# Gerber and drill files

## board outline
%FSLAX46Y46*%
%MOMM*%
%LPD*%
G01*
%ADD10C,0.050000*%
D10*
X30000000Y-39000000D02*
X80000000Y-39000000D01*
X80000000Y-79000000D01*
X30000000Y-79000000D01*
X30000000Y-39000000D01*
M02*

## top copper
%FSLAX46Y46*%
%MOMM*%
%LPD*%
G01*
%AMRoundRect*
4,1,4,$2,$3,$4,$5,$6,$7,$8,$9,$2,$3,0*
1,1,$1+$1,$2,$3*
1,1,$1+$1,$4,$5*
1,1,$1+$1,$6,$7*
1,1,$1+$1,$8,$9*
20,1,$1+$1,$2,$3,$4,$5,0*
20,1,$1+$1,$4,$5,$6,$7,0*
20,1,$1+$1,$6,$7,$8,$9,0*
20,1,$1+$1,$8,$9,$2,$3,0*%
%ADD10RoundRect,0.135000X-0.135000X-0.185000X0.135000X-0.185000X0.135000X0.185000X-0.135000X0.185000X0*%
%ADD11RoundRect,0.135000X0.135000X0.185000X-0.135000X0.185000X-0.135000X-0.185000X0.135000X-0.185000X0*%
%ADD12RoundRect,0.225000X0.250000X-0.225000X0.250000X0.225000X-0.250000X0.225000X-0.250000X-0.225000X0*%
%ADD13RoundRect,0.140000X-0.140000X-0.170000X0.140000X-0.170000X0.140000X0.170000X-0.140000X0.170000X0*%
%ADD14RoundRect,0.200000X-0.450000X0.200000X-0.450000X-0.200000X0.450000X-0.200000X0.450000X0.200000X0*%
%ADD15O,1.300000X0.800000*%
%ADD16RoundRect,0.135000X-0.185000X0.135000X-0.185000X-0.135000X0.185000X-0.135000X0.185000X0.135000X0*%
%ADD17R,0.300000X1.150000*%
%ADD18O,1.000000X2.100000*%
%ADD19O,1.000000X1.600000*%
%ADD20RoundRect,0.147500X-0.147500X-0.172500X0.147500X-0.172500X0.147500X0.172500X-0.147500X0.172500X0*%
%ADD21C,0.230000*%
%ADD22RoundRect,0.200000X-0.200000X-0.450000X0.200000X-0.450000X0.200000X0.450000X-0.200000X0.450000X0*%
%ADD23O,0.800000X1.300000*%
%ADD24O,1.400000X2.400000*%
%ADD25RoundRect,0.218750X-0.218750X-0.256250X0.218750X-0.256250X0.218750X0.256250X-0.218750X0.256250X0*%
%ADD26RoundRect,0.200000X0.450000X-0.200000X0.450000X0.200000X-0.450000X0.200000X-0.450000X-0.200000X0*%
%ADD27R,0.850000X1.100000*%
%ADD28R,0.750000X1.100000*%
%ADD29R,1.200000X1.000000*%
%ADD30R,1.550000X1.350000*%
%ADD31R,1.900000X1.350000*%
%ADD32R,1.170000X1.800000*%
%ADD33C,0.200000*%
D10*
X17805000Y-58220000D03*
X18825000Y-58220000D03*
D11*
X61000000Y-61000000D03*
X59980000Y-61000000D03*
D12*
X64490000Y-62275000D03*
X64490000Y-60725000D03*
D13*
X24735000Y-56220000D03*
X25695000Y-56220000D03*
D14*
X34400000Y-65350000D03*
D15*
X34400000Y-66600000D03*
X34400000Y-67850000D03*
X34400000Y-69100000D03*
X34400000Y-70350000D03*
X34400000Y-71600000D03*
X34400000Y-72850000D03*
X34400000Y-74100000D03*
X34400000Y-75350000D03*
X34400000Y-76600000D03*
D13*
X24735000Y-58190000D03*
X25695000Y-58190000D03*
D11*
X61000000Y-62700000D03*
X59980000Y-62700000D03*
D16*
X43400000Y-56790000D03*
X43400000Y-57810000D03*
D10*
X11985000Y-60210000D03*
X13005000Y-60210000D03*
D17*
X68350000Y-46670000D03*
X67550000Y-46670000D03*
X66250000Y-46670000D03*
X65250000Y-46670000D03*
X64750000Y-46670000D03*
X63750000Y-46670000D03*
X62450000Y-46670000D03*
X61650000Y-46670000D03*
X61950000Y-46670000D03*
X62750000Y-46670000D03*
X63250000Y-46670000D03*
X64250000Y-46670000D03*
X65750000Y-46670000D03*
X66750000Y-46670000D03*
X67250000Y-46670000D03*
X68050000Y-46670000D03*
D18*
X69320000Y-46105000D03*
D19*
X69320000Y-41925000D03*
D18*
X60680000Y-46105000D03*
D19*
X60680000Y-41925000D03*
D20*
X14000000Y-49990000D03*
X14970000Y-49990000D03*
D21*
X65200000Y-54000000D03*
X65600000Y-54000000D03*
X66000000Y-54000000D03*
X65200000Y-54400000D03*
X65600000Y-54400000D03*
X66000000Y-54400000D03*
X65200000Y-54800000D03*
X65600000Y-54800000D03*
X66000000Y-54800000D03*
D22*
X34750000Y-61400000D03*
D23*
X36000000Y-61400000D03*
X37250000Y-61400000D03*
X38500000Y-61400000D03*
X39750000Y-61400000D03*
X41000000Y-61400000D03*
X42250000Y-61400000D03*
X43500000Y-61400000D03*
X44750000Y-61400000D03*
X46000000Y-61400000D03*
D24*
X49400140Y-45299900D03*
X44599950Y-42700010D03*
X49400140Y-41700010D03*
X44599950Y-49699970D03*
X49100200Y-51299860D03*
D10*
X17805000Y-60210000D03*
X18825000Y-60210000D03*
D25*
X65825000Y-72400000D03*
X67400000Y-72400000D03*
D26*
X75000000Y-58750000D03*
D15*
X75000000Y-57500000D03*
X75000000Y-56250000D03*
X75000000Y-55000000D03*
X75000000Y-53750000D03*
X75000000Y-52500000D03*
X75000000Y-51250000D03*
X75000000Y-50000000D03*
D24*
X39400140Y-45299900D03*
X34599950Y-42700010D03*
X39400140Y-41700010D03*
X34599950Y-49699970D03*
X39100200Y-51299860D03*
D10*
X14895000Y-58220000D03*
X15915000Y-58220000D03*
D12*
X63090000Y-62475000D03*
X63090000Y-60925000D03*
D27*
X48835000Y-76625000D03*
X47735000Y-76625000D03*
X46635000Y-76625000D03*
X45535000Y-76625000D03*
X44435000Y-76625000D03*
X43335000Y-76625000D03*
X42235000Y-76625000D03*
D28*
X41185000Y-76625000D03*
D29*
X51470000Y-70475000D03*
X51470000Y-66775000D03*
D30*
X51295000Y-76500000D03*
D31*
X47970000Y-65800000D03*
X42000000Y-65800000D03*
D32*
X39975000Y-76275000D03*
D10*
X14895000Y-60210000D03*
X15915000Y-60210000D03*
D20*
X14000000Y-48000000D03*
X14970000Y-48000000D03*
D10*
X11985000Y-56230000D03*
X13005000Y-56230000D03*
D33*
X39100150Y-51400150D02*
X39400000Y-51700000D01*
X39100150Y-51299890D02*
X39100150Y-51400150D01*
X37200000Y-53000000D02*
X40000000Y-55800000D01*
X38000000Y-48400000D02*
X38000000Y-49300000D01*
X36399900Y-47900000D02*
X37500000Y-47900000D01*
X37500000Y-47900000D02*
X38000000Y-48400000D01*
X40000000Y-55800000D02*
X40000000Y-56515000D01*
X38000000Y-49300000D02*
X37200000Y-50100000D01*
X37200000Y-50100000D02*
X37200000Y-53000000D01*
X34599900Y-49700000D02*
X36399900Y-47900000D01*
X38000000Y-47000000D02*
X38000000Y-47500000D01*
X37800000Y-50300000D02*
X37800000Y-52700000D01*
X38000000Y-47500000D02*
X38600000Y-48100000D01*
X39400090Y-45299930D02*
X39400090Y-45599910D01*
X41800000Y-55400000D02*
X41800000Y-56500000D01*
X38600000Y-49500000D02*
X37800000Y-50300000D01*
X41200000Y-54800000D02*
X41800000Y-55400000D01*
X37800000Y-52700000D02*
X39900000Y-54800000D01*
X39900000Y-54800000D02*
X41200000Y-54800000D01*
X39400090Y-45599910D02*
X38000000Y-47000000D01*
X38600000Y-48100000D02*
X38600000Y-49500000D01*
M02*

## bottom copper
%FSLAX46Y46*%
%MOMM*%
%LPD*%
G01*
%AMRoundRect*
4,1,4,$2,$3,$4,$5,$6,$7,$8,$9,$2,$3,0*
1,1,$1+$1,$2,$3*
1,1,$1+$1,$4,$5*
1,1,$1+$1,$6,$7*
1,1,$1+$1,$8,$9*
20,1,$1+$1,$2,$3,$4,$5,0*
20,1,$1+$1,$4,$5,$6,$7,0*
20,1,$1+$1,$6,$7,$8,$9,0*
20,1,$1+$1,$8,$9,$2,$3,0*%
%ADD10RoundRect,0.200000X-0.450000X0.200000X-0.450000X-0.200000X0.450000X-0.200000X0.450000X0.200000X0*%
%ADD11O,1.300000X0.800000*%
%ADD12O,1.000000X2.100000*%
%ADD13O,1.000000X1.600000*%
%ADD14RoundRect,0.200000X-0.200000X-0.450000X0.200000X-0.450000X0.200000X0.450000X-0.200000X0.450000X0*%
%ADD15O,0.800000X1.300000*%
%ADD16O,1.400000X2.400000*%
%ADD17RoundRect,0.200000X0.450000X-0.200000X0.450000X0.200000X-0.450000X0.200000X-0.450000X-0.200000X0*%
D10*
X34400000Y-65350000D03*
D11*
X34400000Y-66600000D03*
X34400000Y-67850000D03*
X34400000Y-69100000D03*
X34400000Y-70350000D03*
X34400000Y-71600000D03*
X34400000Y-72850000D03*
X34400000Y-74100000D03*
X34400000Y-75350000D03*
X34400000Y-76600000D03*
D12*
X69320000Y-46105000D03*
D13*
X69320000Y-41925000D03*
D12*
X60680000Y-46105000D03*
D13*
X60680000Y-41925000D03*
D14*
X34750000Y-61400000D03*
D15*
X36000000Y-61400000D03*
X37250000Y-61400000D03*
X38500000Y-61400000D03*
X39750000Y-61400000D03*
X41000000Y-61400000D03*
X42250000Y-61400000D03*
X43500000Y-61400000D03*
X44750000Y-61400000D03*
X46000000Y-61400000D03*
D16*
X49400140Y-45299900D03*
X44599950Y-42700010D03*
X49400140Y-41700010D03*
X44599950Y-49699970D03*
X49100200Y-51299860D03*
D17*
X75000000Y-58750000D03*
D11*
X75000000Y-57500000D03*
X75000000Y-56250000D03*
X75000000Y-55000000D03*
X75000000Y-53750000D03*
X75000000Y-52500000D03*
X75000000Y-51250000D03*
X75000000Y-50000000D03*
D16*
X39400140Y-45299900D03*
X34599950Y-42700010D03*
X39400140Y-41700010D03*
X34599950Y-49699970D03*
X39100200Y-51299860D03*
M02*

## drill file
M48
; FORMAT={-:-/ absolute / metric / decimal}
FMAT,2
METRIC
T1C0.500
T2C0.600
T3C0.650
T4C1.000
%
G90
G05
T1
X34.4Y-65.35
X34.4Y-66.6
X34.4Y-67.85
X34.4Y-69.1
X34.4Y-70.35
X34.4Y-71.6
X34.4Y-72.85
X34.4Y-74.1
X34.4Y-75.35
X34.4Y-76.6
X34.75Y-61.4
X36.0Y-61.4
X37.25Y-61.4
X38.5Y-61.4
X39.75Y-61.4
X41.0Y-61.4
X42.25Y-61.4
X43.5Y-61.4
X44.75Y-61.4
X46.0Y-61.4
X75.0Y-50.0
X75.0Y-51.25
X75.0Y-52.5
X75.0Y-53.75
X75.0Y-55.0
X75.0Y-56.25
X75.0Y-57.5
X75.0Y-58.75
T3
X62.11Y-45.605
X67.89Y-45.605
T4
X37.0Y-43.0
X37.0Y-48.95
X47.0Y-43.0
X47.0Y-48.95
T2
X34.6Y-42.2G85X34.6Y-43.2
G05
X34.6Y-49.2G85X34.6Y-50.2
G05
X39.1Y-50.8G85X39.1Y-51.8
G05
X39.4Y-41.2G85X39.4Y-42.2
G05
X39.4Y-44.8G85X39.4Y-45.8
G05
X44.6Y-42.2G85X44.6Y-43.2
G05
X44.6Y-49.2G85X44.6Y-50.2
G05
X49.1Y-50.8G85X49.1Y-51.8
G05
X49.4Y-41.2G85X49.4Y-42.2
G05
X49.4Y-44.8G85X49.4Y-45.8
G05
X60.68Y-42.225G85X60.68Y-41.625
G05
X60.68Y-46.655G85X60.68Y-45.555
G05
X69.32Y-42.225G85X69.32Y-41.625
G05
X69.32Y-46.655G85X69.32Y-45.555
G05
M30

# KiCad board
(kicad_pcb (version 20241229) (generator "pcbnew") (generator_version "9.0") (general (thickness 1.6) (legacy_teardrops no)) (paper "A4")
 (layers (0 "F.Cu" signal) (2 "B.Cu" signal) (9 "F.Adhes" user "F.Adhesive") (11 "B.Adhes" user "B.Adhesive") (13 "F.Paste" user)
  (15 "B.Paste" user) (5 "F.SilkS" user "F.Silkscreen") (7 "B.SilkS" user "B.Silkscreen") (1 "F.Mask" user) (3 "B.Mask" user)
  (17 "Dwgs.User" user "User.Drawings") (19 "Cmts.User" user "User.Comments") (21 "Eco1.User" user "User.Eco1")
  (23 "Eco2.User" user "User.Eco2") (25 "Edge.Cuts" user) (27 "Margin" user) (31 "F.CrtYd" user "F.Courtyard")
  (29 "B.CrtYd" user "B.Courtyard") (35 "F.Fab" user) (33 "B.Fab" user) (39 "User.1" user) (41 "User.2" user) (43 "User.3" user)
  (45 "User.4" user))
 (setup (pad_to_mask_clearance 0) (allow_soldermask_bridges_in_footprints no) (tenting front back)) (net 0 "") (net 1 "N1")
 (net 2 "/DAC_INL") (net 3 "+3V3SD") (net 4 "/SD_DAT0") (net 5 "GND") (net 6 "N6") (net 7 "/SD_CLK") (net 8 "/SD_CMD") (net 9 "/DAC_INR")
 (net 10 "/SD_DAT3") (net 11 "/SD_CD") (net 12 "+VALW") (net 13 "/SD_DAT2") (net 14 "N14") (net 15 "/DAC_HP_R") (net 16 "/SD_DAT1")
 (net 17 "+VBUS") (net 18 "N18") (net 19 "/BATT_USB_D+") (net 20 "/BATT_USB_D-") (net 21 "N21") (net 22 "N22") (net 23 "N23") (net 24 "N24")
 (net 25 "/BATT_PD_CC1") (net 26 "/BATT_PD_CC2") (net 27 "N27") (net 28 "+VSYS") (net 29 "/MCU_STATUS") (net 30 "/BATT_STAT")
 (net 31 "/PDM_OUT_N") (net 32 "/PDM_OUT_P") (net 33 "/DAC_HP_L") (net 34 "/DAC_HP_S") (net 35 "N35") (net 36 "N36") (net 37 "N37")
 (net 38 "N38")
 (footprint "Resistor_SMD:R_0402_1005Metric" (layer "F.Cu") (at 18.315 58.22)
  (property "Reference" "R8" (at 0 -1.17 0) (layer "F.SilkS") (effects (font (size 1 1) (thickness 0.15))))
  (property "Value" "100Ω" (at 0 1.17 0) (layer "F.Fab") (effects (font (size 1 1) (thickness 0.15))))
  (pad "1" smd roundrect (at -0.51 0) (size 0.54 0.64) (layers "F.Cu" "F.Mask" "F.Paste") (roundrect_rratio 0.25) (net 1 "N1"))
  (pad "2" smd roundrect (at 0.51 0) (size 0.54 0.64) (layers "F.Cu" "F.Mask" "F.Paste") (roundrect_rratio 0.25) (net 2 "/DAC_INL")))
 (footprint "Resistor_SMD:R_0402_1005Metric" (layer "F.Cu") (at 60.49 61 180)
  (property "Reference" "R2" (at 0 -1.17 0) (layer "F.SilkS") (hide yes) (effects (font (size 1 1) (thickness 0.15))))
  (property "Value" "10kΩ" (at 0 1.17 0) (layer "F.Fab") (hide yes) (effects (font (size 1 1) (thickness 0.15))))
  (pad "1" smd roundrect (at -0.51 0 180) (size 0.54 0.64) (layers "F.Cu" "F.Mask" "F.Paste") (roundrect_rratio 0.25) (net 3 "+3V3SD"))
  (pad "2" smd roundrect (at 0.51 0 180) (size 0.54 0.64) (layers "F.Cu" "F.Mask" "F.Paste") (roundrect_rratio 0.25) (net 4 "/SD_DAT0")))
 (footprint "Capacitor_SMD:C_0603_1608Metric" (layer "F.Cu") (at 64.49 61.5 90)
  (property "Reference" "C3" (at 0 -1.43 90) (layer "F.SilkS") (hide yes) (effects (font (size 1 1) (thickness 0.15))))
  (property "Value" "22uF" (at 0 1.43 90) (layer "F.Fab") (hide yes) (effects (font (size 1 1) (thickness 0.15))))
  (pad "1" smd roundrect (at -0.775 0 90) (size 0.9 0.95) (layers "F.Cu" "F.Mask" "F.Paste") (roundrect_rratio 0.25) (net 3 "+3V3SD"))
  (pad "2" smd roundrect (at 0.775 0 90) (size 0.9 0.95) (layers "F.Cu" "F.Mask" "F.Paste") (roundrect_rratio 0.25) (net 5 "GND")))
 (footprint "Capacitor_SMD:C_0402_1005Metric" (layer "F.Cu") (at 25.215 56.22)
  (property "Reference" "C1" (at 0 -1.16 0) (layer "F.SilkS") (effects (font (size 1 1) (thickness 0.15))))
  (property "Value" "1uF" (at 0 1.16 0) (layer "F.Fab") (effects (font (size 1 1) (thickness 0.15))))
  (pad "1" smd roundrect (at -0.48 0) (size 0.56 0.62) (layers "F.Cu" "F.Mask" "F.Paste") (roundrect_rratio 0.25) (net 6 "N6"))
  (pad "2" smd roundrect (at 0.48 0) (size 0.56 0.62) (layers "F.Cu" "F.Mask" "F.Paste") (roundrect_rratio 0.25) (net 5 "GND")))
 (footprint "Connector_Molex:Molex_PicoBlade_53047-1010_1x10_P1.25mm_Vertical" (layer "F.Cu") (at 34.4 65.35 -90)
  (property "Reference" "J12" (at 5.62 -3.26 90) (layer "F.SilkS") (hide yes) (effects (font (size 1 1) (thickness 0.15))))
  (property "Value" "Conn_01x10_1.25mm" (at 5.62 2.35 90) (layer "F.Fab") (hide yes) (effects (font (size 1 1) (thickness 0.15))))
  (pad "1" thru_hole roundrect (at 0 0 270) (size 0.8 1.3) (drill 0.5) (layers "*.Cu" "*.Mask") (remove_unused_layers no)
   (roundrect_rratio 0.25) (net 5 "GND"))
  (pad "2" thru_hole oval (at 1.25 0 270) (size 0.8 1.3) (drill 0.5) (layers "*.Cu" "*.Mask") (remove_unused_layers no) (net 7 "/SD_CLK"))
  (pad "3" thru_hole oval (at 2.5 0 270) (size 0.8 1.3) (drill 0.5) (layers "*.Cu" "*.Mask") (remove_unused_layers no) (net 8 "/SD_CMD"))
  (pad "4" thru_hole oval (at 3.75 0 270) (size 0.8 1.3) (drill 0.5) (layers "*.Cu" "*.Mask") (remove_unused_layers no) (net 3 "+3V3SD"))
  (pad "5" thru_hole oval (at 5 0 270) (size 0.8 1.3) (drill 0.5) (layers "*.Cu" "*.Mask") (remove_unused_layers no) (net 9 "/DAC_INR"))
  (pad "6" thru_hole oval (at 6.25 0 270) (size 0.8 1.3) (drill 0.5) (layers "*.Cu" "*.Mask") (remove_unused_layers no) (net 2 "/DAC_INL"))
  (pad "7" thru_hole oval (at 7.5 0 270) (size 0.8 1.3) (drill 0.5) (layers "*.Cu" "*.Mask") (remove_unused_layers no) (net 5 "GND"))
  (pad "8" thru_hole oval (at 8.75 0 270) (size 0.8 1.3) (drill 0.5) (layers "*.Cu" "*.Mask") (remove_unused_layers no) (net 4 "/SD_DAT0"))
  (pad "9" thru_hole oval (at 10 0 270) (size 0.8 1.3) (drill 0.5) (layers "*.Cu" "*.Mask") (remove_unused_layers no) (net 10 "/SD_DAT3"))
  (pad "10" thru_hole oval (at 11.25 0 270) (size 0.8 1.3) (drill 0.5) (layers "*.Cu" "*.Mask") (remove_unused_layers no) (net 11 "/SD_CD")))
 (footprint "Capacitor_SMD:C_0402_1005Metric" (layer "F.Cu") (at 25.215 58.19)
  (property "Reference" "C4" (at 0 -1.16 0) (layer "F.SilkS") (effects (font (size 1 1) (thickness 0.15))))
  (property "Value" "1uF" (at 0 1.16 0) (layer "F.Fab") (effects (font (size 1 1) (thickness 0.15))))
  (pad "1" smd roundrect (at -0.48 0) (size 0.56 0.62) (layers "F.Cu" "F.Mask" "F.Paste") (roundrect_rratio 0.25) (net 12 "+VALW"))
  (pad "2" smd roundrect (at 0.48 0) (size 0.56 0.62) (layers "F.Cu" "F.Mask" "F.Paste") (roundrect_rratio 0.25) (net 5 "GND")))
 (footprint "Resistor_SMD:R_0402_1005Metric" (layer "F.Cu") (at 60.49 62.7 180)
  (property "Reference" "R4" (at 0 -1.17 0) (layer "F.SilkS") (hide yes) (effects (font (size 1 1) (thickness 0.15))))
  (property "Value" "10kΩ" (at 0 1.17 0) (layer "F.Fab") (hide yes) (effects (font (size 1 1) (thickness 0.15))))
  (pad "1" smd roundrect (at -0.51 0 180) (size 0.54 0.64) (layers "F.Cu" "F.Mask" "F.Paste") (roundrect_rratio 0.25) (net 3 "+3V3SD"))
  (pad "2" smd roundrect (at 0.51 0 180) (size 0.54 0.64) (layers "F.Cu" "F.Mask" "F.Paste") (roundrect_rratio 0.25) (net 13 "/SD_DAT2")))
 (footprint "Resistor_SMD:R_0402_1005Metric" (layer "F.Cu") (at 43.4 57.3 -90)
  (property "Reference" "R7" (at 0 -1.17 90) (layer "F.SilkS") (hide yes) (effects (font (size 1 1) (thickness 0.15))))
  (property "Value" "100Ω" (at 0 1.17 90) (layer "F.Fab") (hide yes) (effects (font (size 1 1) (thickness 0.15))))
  (pad "1" smd roundrect (at -0.51 0 270) (size 0.54 0.64) (layers "F.Cu" "F.Mask" "F.Paste") (roundrect_rratio 0.25) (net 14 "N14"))
  (pad "2" smd roundrect (at 0.51 0 270) (size 0.54 0.64) (layers "F.Cu" "F.Mask" "F.Paste") (roundrect_rratio 0.25) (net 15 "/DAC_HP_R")))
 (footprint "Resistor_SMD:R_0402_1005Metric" (layer "F.Cu") (at 12.495 60.21)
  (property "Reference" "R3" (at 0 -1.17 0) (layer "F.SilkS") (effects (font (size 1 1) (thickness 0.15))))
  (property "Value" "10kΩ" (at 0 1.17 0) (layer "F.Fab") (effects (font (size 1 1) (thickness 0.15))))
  (pad "1" smd roundrect (at -0.51 0) (size 0.54 0.64) (layers "F.Cu" "F.Mask" "F.Paste") (roundrect_rratio 0.25) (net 3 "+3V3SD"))
  (pad "2" smd roundrect (at 0.51 0) (size 0.54 0.64) (layers "F.Cu" "F.Mask" "F.Paste") (roundrect_rratio 0.25) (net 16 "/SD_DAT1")))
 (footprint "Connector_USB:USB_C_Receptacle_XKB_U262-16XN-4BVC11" (layer "F.Cu") (at 65 43 180)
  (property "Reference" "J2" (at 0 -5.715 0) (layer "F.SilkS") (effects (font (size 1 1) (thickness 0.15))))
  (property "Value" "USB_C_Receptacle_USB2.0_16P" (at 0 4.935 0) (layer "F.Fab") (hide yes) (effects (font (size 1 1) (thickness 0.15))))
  (pad "" np_thru_hole circle (at -2.89 -2.605 180) (size 0.65 0.65) (drill 0.65) (layers "*.Cu" "*.Mask"))
  (pad "" np_thru_hole circle (at 2.89 -2.605 180) (size 0.65 0.65) (drill 0.65) (layers "*.Cu" "*.Mask"))
  (pad "A1" smd rect (at -3.35 -3.67 180) (size 0.3 1.15) (layers "F.Cu" "F.Mask" "F.Paste") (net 5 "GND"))
  (pad "A4" smd rect (at -2.55 -3.67 180) (size 0.3 1.15) (layers "F.Cu" "F.Mask" "F.Paste") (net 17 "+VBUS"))
  (pad "A5" smd rect (at -1.25 -3.67 180) (size 0.3 1.15) (layers "F.Cu" "F.Mask" "F.Paste") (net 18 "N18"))
  (pad "A6" smd rect (at -0.25 -3.67 180) (size 0.3 1.15) (layers "F.Cu" "F.Mask" "F.Paste") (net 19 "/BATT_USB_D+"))
  (pad "A7" smd rect (at 0.25 -3.67 180) (size 0.3 1.15) (layers "F.Cu" "F.Mask" "F.Paste") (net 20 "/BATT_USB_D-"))
  (pad "A8" smd rect (at 1.25 -3.67 180) (size 0.3 1.15) (layers "F.Cu" "F.Mask" "F.Paste") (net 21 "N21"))
  (pad "A9" smd rect (at 2.55 -3.67 180) (size 0.3 1.15) (layers "F.Cu" "F.Mask" "F.Paste") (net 17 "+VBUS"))
  (pad "A12" smd rect (at 3.35 -3.67 180) (size 0.3 1.15) (layers "F.Cu" "F.Mask" "F.Paste") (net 5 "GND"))
  (pad "B1" smd rect (at 3.05 -3.67 180) (size 0.3 1.15) (layers "F.Cu" "F.Mask" "F.Paste") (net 5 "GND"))
  (pad "B4" smd rect (at 2.25 -3.67 180) (size 0.3 1.15) (layers "F.Cu" "F.Mask" "F.Paste") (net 17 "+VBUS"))
  (pad "B5" smd rect (at 1.75 -3.67 180) (size 0.3 1.15) (layers "F.Cu" "F.Mask" "F.Paste") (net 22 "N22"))
  (pad "B6" smd rect (at 0.75 -3.67 180) (size 0.3 1.15) (layers "F.Cu" "F.Mask" "F.Paste") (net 19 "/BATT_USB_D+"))
  (pad "B7" smd rect (at -0.75 -3.67 180) (size 0.3 1.15) (layers "F.Cu" "F.Mask" "F.Paste") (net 20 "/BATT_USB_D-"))
  (pad "B8" smd rect (at -1.75 -3.67 180) (size 0.3 1.15) (layers "F.Cu" "F.Mask" "F.Paste") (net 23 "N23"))
  (pad "B9" smd rect (at -2.25 -3.67 180) (size 0.3 1.15) (layers "F.Cu" "F.Mask" "F.Paste") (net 17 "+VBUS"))
  (pad "B12" smd rect (at -3.05 -3.67 180) (size 0.3 1.15) (layers "F.Cu" "F.Mask" "F.Paste") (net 5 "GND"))
  (pad "S1" thru_hole oval (at -4.32 -3.105 180) (size 1 2.1) (drill oval 0.6 1.7) (layers "*.Cu" "*.Mask") (remove_unused_layers no)
   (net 5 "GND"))
  (pad "S1" thru_hole oval (at -4.32 1.075 180) (size 1 1.6) (drill oval 0.6 1.2) (layers "*.Cu" "*.Mask") (remove_unused_layers no)
   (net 5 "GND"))
  (pad "S1" thru_hole oval (at 4.32 -3.105 180) (size 1 2.1) (drill oval 0.6 1.7) (layers "*.Cu" "*.Mask") (remove_unused_layers no)
   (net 5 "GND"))
  (pad "S1" thru_hole oval (at 4.32 1.075 180) (size 1 1.6) (drill oval 0.6 1.2) (layers "*.Cu" "*.Mask") (remove_unused_layers no)
   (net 5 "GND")))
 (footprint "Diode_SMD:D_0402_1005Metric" (layer "F.Cu") (at 14.485 49.99)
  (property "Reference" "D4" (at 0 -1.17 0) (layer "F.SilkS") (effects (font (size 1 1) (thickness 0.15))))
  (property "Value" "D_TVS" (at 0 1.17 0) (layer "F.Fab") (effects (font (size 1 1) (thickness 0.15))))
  (pad "1" smd roundrect (at -0.485 0) (size 0.59 0.64) (layers "F.Cu" "F.Mask" "F.Paste") (roundrect_rratio 0.25) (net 5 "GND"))
  (pad "2" smd roundrect (at 0.485 0) (size 0.59 0.64) (layers "F.Cu" "F.Mask" "F.Paste") (roundrect_rratio 0.25) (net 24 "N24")))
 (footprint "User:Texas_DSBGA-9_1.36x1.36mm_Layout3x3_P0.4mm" (layer "F.Cu") (at 65.6 54.4)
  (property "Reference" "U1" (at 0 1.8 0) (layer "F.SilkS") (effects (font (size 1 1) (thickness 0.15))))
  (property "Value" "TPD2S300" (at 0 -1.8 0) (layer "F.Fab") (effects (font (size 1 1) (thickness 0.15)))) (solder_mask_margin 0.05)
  (pad "A1" smd circle (at -0.4 -0.4) (size 0.23 0.23) (layers "F.Cu" "F.Paste") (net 18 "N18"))
  (pad "A2" smd circle (at 0 -0.4) (size 0.23 0.23) (layers "F.Cu" "F.Paste") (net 6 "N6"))
  (pad "A3" smd circle (at 0.4 -0.4) (size 0.23 0.23) (layers "F.Cu" "F.Paste") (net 22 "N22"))
  (pad "B1" smd circle (at -0.4 0) (size 0.23 0.23) (layers "F.Cu" "F.Paste") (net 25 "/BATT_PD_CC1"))
  (pad "B2" smd circle (at 0 0) (size 0.23 0.23) (layers "F.Cu" "F.Paste") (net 5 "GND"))
  (pad "B3" smd circle (at 0.4 0) (size 0.23 0.23) (layers "F.Cu" "F.Paste") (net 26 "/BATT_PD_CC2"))
  (pad "C1" smd circle (at -0.4 0.4) (size 0.23 0.23) (layers "F.Cu" "F.Paste") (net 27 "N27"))
  (pad "C2" smd circle (at 0 0.4) (size 0.23 0.23) (layers "F.Cu" "F.Paste") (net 12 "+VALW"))
  (pad "C3" smd circle (at 0.4 0.4) (size 0.23 0.23) (layers "F.Cu" "F.Paste") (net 12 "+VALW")))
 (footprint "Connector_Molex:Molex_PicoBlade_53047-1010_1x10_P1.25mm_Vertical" (layer "F.Cu") (at 34.75 61.4)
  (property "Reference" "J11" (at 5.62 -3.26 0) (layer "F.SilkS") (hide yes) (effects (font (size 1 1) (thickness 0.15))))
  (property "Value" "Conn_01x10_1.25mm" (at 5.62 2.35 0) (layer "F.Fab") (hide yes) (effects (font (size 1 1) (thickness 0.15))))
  (pad "1" thru_hole roundrect (at 0 0) (size 0.8 1.3) (drill 0.5) (layers "*.Cu" "*.Mask") (remove_unused_layers no)
   (roundrect_rratio 0.25) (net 5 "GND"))
  (pad "2" thru_hole oval (at 1.25 0) (size 0.8 1.3) (drill 0.5) (layers "*.Cu" "*.Mask") (remove_unused_layers no) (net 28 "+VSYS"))
  (pad "3" thru_hole oval (at 2.5 0) (size 0.8 1.3) (drill 0.5) (layers "*.Cu" "*.Mask") (remove_unused_layers no) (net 12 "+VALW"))
  (pad "4" thru_hole oval (at 3.75 0) (size 0.8 1.3) (drill 0.5) (layers "*.Cu" "*.Mask") (remove_unused_layers no) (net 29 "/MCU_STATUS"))
  (pad "5" thru_hole oval (at 5 0) (size 0.8 1.3) (drill 0.5) (layers "*.Cu" "*.Mask") (remove_unused_layers no) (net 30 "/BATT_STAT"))
  (pad "6" thru_hole oval (at 6.25 0) (size 0.8 1.3) (drill 0.5) (layers "*.Cu" "*.Mask") (remove_unused_layers no) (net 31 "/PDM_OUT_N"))
  (pad "7" thru_hole oval (at 7.5 0) (size 0.8 1.3) (drill 0.5) (layers "*.Cu" "*.Mask") (remove_unused_layers no) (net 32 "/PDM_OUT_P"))
  (pad "8" thru_hole oval (at 8.75 0) (size 0.8 1.3) (drill 0.5) (layers "*.Cu" "*.Mask") (remove_unused_layers no) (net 15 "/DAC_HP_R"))
  (pad "9" thru_hole oval (at 10 0) (size 0.8 1.3) (drill 0.5) (layers "*.Cu" "*.Mask") (remove_unused_layers no) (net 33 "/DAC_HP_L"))
  (pad "10" thru_hole oval (at 11.25 0) (size 0.8 1.3) (drill 0.5) (layers "*.Cu" "*.Mask") (remove_unused_layers no) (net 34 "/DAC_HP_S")))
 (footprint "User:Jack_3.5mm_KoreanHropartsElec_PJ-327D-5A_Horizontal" (layer "F.Cu") (at 47 46.5)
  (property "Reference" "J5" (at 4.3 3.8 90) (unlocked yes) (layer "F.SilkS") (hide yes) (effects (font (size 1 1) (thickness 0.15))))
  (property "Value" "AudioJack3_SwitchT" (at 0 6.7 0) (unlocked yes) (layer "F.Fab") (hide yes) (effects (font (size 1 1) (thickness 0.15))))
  (pad "" np_thru_hole circle (at 0 -3.5) (size 1 1) (drill 1) (layers "*.Cu" "*.Mask"))
  (pad "" np_thru_hole circle (at 0 2.45) (size 1 1) (drill 1) (layers "*.Cu" "*.Mask"))
  (pad "R" thru_hole oval (at 2.40009 -1.20007) (size 1.4 2.4) (drill oval 0.6 1.6 (offset 0.00005 -0.00003)) (layers "*.Cu" "*.Mask")
   (remove_unused_layers no) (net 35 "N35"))
  (pad "S" thru_hole oval (at -2.4001 -3.79996) (size 1.4 2.4) (drill oval 0.6 1.6 (offset 0.00005 -0.00003)) (layers "*.Cu" "*.Mask")
   (remove_unused_layers no) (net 5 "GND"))
  (pad "S" thru_hole oval (at 2.40009 -4.79996) (size 1.4 2.4) (drill oval 0.6 1.6 (offset 0.00005 -0.00003)) (layers "*.Cu" "*.Mask")
   (remove_unused_layers no) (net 5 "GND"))
  (pad "T" thru_hole oval (at -2.4001 3.2) (size 1.4 2.4) (drill oval 0.6 1.6 (offset 0.00005 -0.00003)) (layers "*.Cu" "*.Mask")
   (remove_unused_layers no) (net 1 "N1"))
  (pad "TN" thru_hole oval (at 2.10015 4.79989) (size 1.4 2.4) (drill oval 0.6 1.6 (offset 0.00005 -0.00003)) (layers "*.Cu" "*.Mask")
   (remove_unused_layers no) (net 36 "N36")))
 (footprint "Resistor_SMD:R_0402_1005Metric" (layer "F.Cu") (at 18.315 60.21)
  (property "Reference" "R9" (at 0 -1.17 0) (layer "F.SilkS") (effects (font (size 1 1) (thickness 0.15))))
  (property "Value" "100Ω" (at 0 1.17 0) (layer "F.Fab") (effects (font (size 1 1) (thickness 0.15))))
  (pad "1" smd roundrect (at -0.51 0) (size 0.54 0.64) (layers "F.Cu" "F.Mask" "F.Paste") (roundrect_rratio 0.25) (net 35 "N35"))
  (pad "2" smd roundrect (at 0.51 0) (size 0.54 0.64) (layers "F.Cu" "F.Mask" "F.Paste") (roundrect_rratio 0.25) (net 9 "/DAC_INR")))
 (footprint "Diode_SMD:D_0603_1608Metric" (layer "F.Cu") (at 66.6125 72.4)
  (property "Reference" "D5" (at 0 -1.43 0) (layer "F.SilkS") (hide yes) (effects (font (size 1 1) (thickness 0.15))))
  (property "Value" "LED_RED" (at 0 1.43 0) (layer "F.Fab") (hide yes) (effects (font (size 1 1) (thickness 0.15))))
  (pad "1" smd roundrect (at -0.7875 0) (size 0.875 0.95) (layers "F.Cu" "F.Mask" "F.Paste") (roundrect_rratio 0.25) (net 30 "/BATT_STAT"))
  (pad "2" smd roundrect (at 0.7875 0) (size 0.875 0.95) (layers "F.Cu" "F.Mask" "F.Paste") (roundrect_rratio 0.25) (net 12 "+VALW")))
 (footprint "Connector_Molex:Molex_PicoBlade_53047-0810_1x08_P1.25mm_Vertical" (layer "F.Cu") (at 75 58.75 90)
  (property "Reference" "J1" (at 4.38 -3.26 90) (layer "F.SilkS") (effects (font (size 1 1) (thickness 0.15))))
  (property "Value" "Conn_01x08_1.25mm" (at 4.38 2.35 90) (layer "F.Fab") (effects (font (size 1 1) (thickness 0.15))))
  (pad "1" thru_hole roundrect (at 0 0 90) (size 0.8 1.3) (drill 0.5) (layers "*.Cu" "*.Mask") (remove_unused_layers no)
   (roundrect_rratio 0.25) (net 17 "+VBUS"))
  (pad "2" thru_hole oval (at 1.25 0 90) (size 0.8 1.3) (drill 0.5) (layers "*.Cu" "*.Mask") (remove_unused_layers no) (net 17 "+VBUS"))
  (pad "3" thru_hole oval (at 2.5 0 90) (size 0.8 1.3) (drill 0.5) (layers "*.Cu" "*.Mask") (remove_unused_layers no) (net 5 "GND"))
  (pad "4" thru_hole oval (at 3.75 0 90) (size 0.8 1.3) (drill 0.5) (layers "*.Cu" "*.Mask") (remove_unused_layers no) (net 5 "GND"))
  (pad "5" thru_hole oval (at 5 0 90) (size 0.8 1.3) (drill 0.5) (layers "*.Cu" "*.Mask") (remove_unused_layers no) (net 26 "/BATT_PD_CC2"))
  (pad "6" thru_hole oval (at 6.25 0 90) (size 0.8 1.3) (drill 0.5) (layers "*.Cu" "*.Mask") (remove_unused_layers no)
   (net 25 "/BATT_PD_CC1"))
  (pad "7" thru_hole oval (at 7.5 0 90) (size 0.8 1.3) (drill 0.5) (layers "*.Cu" "*.Mask") (remove_unused_layers no)
   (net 19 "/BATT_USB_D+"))
  (pad "8" thru_hole oval (at 8.75 0 90) (size 0.8 1.3) (drill 0.5) (layers "*.Cu" "*.Mask") (remove_unused_layers no)
   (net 20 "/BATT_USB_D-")))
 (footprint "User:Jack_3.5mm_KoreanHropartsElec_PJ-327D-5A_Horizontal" (layer "F.Cu") (at 37 46.5)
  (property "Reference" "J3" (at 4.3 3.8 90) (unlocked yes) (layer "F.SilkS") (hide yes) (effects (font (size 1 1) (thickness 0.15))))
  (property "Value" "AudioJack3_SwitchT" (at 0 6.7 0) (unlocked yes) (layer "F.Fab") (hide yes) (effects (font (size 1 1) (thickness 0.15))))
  (pad "" np_thru_hole circle (at 0 -3.5) (size 1 1) (drill 1) (layers "*.Cu" "*.Mask"))
  (pad "" np_thru_hole circle (at 0 2.45) (size 1 1) (drill 1) (layers "*.Cu" "*.Mask"))
  (pad "R" thru_hole oval (at 2.40009 -1.20007) (size 1.4 2.4) (drill oval 0.6 1.6 (offset 0.00005 -0.00003)) (layers "*.Cu" "*.Mask")
   (remove_unused_layers no) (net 14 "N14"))
  (pad "S" thru_hole oval (at -2.4001 -3.79996) (size 1.4 2.4) (drill oval 0.6 1.6 (offset 0.00005 -0.00003)) (layers "*.Cu" "*.Mask")
   (remove_unused_layers no) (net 5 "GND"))
  (pad "S" thru_hole oval (at 2.40009 -4.79996) (size 1.4 2.4) (drill oval 0.6 1.6 (offset 0.00005 -0.00003)) (layers "*.Cu" "*.Mask")
   (remove_unused_layers no) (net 5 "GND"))
  (pad "T" thru_hole oval (at -2.4001 3.2) (size 1.4 2.4) (drill oval 0.6 1.6 (offset 0.00005 -0.00003)) (layers "*.Cu" "*.Mask")
   (remove_unused_layers no) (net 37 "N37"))
  (pad "TN" thru_hole oval (at 2.10015 4.79989) (size 1.4 2.4) (drill oval 0.6 1.6 (offset 0.00005 -0.00003)) (layers "*.Cu" "*.Mask")
   (remove_unused_layers no) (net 34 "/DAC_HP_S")))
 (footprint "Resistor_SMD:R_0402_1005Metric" (layer "F.Cu") (at 15.405 58.22)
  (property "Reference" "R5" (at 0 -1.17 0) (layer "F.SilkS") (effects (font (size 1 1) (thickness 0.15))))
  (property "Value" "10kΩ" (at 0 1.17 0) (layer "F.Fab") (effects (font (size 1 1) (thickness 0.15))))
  (pad "1" smd roundrect (at -0.51 0) (size 0.54 0.64) (layers "F.Cu" "F.Mask" "F.Paste") (roundrect_rratio 0.25) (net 3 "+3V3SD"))
  (pad "2" smd roundrect (at 0.51 0) (size 0.54 0.64) (layers "F.Cu" "F.Mask" "F.Paste") (roundrect_rratio 0.25) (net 8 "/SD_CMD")))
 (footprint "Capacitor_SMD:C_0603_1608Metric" (layer "F.Cu") (at 63.09 61.7 90)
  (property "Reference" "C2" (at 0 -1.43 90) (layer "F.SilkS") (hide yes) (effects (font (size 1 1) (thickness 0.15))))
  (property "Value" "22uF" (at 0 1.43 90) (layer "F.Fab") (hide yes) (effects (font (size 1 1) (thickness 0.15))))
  (pad "1" smd roundrect (at -0.775 0 90) (size 0.9 0.95) (layers "F.Cu" "F.Mask" "F.Paste") (roundrect_rratio 0.25) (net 3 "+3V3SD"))
  (pad "2" smd roundrect (at 0.775 0 90) (size 0.9 0.95) (layers "F.Cu" "F.Mask" "F.Paste") (roundrect_rratio 0.25) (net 5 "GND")))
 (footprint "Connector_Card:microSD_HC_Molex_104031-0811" (layer "F.Cu") (at 45.73 71.175 180)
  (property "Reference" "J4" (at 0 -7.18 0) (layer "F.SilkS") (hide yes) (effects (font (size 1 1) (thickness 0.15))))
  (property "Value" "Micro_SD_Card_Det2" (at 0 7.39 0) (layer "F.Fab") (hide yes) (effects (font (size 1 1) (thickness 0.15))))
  (pad "1" smd rect (at -3.105 -5.45 180) (size 0.85 1.1) (layers "F.Cu" "F.Mask" "F.Paste") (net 13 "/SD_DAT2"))
  (pad "2" smd rect (at -2.005 -5.45 180) (size 0.85 1.1) (layers "F.Cu" "F.Mask" "F.Paste") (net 10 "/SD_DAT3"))
  (pad "3" smd rect (at -0.905 -5.45 180) (size 0.85 1.1) (layers "F.Cu" "F.Mask" "F.Paste") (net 8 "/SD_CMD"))
  (pad "4" smd rect (at 0.195 -5.45 180) (size 0.85 1.1) (layers "F.Cu" "F.Mask" "F.Paste") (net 3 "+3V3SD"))
  (pad "5" smd rect (at 1.295 -5.45 180) (size 0.85 1.1) (layers "F.Cu" "F.Mask" "F.Paste") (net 7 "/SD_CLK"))
  (pad "6" smd rect (at 2.395 -5.45 180) (size 0.85 1.1) (layers "F.Cu" "F.Mask" "F.Paste") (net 5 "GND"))
  (pad "7" smd rect (at 3.495 -5.45 180) (size 0.85 1.1) (layers "F.Cu" "F.Mask" "F.Paste") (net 4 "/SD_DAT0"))
  (pad "8" smd rect (at 4.545 -5.45 180) (size 0.75 1.1) (layers "F.Cu" "F.Mask" "F.Paste") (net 16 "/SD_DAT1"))
  (pad "9" smd rect (at -5.74 0.7 180) (size 1.2 1) (layers "F.Cu" "F.Mask" "F.Paste") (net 3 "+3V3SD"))
  (pad "10" smd rect (at -5.74 4.4 180) (size 1.2 1) (layers "F.Cu" "F.Mask" "F.Paste") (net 11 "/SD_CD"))
  (pad "11" smd rect (at -5.565 -5.325 180) (size 1.55 1.35) (layers "F.Cu" "F.Mask" "F.Paste") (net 5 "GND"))
  (pad "11" smd rect (at -2.24 5.375 180) (size 1.9 1.35) (layers "F.Cu" "F.Mask" "F.Paste") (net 5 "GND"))
  (pad "11" smd rect (at 3.73 5.375 180) (size 1.9 1.35) (layers "F.Cu" "F.Mask" "F.Paste") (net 5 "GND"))
  (pad "11" smd rect (at 5.755 -5.1 180) (size 1.17 1.8) (layers "F.Cu" "F.Mask" "F.Paste") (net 5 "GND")))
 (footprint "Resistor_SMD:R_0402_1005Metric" (layer "F.Cu") (at 15.405 60.21)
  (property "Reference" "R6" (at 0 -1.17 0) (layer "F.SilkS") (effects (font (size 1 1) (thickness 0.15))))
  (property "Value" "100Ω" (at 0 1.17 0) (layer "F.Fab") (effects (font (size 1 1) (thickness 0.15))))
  (pad "1" smd roundrect (at -0.51 0) (size 0.54 0.64) (layers "F.Cu" "F.Mask" "F.Paste") (roundrect_rratio 0.25) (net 37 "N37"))
  (pad "2" smd roundrect (at 0.51 0) (size 0.54 0.64) (layers "F.Cu" "F.Mask" "F.Paste") (roundrect_rratio 0.25) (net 33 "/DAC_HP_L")))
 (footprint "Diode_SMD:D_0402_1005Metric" (layer "F.Cu") (at 14.485 48)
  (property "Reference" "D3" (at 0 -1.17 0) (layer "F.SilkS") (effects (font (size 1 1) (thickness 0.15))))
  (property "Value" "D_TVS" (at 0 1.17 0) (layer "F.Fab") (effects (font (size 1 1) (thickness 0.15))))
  (pad "1" smd roundrect (at -0.485 0) (size 0.59 0.64) (layers "F.Cu" "F.Mask" "F.Paste") (roundrect_rratio 0.25) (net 5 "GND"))
  (pad "2" smd roundrect (at 0.485 0) (size 0.59 0.64) (layers "F.Cu" "F.Mask" "F.Paste") (roundrect_rratio 0.25) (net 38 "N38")))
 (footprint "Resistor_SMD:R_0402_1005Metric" (layer "F.Cu") (at 12.495 56.23)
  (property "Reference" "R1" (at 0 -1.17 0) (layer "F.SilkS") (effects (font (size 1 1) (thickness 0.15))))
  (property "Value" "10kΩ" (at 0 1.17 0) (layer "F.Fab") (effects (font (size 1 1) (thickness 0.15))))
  (pad "1" smd roundrect (at -0.51 0) (size 0.54 0.64) (layers "F.Cu" "F.Mask" "F.Paste") (roundrect_rratio 0.25) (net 11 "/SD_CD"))
  (pad "2" smd roundrect (at 0.51 0) (size 0.54 0.64) (layers "F.Cu" "F.Mask" "F.Paste") (roundrect_rratio 0.25) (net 5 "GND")))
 (gr_rect (start 30 39) (end 80 79) (stroke (width 0.05) (type default)) (fill no) (layer "Edge.Cuts"))
 (segment (start 39.10015 51.40015) (end 39.4 51.7) (width 0.2) (layer "F.Cu") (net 34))
 (segment (start 39.10015 51.29989) (end 39.10015 51.40015) (width 0.2) (layer "F.Cu") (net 34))
 (segment (start 37.2 53) (end 40 55.8) (width 0.2) (layer "F.Cu") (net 37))
 (segment (start 38 48.4) (end 38 49.3) (width 0.2) (layer "F.Cu") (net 37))
 (segment (start 36.3999 47.9) (end 37.5 47.9) (width 0.2) (layer "F.Cu") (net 37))
 (segment (start 37.5 47.9) (end 38 48.4) (width 0.2) (layer "F.Cu") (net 37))
 (segment (start 40 55.8) (end 40 56.515) (width 0.2) (layer "F.Cu") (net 37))
 (segment (start 38 49.3) (end 37.2 50.1) (width 0.2) (layer "F.Cu") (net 37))
 (segment (start 37.2 50.1) (end 37.2 53) (width 0.2) (layer "F.Cu") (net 37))
 (segment (start 34.5999 49.7) (end 36.3999 47.9) (width 0.2) (layer "F.Cu") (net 37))
 (segment (start 38 47) (end 38 47.5) (width 0.2) (layer "F.Cu") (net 14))
 (segment (start 37.8 50.3) (end 37.8 52.7) (width 0.2) (layer "F.Cu") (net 14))
 (segment (start 38 47.5) (end 38.6 48.1) (width 0.2) (layer "F.Cu") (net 14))
 (segment (start 39.40009 45.29993) (end 39.40009 45.59991) (width 0.2) (layer "F.Cu") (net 14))
 (segment (start 41.8 55.4) (end 41.8 56.5) (width 0.2) (layer "F.Cu") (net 14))
 (segment (start 38.6 49.5) (end 37.8 50.3) (width 0.2) (layer "F.Cu") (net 14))
 (segment (start 41.2 54.8) (end 41.8 55.4) (width 0.2) (layer "F.Cu") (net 14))
 (segment (start 37.8 52.7) (end 39.9 54.8) (width 0.2) (layer "F.Cu") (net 14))
 (segment (start 39.9 54.8) (end 41.2 54.8) (width 0.2) (layer "F.Cu") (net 14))
 (segment (start 39.40009 45.59991) (end 38 47) (width 0.2) (layer "F.Cu") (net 14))
 (segment (start 38.6 48.1) (end 38.6 49.5) (width 0.2) (layer "F.Cu") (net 14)))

